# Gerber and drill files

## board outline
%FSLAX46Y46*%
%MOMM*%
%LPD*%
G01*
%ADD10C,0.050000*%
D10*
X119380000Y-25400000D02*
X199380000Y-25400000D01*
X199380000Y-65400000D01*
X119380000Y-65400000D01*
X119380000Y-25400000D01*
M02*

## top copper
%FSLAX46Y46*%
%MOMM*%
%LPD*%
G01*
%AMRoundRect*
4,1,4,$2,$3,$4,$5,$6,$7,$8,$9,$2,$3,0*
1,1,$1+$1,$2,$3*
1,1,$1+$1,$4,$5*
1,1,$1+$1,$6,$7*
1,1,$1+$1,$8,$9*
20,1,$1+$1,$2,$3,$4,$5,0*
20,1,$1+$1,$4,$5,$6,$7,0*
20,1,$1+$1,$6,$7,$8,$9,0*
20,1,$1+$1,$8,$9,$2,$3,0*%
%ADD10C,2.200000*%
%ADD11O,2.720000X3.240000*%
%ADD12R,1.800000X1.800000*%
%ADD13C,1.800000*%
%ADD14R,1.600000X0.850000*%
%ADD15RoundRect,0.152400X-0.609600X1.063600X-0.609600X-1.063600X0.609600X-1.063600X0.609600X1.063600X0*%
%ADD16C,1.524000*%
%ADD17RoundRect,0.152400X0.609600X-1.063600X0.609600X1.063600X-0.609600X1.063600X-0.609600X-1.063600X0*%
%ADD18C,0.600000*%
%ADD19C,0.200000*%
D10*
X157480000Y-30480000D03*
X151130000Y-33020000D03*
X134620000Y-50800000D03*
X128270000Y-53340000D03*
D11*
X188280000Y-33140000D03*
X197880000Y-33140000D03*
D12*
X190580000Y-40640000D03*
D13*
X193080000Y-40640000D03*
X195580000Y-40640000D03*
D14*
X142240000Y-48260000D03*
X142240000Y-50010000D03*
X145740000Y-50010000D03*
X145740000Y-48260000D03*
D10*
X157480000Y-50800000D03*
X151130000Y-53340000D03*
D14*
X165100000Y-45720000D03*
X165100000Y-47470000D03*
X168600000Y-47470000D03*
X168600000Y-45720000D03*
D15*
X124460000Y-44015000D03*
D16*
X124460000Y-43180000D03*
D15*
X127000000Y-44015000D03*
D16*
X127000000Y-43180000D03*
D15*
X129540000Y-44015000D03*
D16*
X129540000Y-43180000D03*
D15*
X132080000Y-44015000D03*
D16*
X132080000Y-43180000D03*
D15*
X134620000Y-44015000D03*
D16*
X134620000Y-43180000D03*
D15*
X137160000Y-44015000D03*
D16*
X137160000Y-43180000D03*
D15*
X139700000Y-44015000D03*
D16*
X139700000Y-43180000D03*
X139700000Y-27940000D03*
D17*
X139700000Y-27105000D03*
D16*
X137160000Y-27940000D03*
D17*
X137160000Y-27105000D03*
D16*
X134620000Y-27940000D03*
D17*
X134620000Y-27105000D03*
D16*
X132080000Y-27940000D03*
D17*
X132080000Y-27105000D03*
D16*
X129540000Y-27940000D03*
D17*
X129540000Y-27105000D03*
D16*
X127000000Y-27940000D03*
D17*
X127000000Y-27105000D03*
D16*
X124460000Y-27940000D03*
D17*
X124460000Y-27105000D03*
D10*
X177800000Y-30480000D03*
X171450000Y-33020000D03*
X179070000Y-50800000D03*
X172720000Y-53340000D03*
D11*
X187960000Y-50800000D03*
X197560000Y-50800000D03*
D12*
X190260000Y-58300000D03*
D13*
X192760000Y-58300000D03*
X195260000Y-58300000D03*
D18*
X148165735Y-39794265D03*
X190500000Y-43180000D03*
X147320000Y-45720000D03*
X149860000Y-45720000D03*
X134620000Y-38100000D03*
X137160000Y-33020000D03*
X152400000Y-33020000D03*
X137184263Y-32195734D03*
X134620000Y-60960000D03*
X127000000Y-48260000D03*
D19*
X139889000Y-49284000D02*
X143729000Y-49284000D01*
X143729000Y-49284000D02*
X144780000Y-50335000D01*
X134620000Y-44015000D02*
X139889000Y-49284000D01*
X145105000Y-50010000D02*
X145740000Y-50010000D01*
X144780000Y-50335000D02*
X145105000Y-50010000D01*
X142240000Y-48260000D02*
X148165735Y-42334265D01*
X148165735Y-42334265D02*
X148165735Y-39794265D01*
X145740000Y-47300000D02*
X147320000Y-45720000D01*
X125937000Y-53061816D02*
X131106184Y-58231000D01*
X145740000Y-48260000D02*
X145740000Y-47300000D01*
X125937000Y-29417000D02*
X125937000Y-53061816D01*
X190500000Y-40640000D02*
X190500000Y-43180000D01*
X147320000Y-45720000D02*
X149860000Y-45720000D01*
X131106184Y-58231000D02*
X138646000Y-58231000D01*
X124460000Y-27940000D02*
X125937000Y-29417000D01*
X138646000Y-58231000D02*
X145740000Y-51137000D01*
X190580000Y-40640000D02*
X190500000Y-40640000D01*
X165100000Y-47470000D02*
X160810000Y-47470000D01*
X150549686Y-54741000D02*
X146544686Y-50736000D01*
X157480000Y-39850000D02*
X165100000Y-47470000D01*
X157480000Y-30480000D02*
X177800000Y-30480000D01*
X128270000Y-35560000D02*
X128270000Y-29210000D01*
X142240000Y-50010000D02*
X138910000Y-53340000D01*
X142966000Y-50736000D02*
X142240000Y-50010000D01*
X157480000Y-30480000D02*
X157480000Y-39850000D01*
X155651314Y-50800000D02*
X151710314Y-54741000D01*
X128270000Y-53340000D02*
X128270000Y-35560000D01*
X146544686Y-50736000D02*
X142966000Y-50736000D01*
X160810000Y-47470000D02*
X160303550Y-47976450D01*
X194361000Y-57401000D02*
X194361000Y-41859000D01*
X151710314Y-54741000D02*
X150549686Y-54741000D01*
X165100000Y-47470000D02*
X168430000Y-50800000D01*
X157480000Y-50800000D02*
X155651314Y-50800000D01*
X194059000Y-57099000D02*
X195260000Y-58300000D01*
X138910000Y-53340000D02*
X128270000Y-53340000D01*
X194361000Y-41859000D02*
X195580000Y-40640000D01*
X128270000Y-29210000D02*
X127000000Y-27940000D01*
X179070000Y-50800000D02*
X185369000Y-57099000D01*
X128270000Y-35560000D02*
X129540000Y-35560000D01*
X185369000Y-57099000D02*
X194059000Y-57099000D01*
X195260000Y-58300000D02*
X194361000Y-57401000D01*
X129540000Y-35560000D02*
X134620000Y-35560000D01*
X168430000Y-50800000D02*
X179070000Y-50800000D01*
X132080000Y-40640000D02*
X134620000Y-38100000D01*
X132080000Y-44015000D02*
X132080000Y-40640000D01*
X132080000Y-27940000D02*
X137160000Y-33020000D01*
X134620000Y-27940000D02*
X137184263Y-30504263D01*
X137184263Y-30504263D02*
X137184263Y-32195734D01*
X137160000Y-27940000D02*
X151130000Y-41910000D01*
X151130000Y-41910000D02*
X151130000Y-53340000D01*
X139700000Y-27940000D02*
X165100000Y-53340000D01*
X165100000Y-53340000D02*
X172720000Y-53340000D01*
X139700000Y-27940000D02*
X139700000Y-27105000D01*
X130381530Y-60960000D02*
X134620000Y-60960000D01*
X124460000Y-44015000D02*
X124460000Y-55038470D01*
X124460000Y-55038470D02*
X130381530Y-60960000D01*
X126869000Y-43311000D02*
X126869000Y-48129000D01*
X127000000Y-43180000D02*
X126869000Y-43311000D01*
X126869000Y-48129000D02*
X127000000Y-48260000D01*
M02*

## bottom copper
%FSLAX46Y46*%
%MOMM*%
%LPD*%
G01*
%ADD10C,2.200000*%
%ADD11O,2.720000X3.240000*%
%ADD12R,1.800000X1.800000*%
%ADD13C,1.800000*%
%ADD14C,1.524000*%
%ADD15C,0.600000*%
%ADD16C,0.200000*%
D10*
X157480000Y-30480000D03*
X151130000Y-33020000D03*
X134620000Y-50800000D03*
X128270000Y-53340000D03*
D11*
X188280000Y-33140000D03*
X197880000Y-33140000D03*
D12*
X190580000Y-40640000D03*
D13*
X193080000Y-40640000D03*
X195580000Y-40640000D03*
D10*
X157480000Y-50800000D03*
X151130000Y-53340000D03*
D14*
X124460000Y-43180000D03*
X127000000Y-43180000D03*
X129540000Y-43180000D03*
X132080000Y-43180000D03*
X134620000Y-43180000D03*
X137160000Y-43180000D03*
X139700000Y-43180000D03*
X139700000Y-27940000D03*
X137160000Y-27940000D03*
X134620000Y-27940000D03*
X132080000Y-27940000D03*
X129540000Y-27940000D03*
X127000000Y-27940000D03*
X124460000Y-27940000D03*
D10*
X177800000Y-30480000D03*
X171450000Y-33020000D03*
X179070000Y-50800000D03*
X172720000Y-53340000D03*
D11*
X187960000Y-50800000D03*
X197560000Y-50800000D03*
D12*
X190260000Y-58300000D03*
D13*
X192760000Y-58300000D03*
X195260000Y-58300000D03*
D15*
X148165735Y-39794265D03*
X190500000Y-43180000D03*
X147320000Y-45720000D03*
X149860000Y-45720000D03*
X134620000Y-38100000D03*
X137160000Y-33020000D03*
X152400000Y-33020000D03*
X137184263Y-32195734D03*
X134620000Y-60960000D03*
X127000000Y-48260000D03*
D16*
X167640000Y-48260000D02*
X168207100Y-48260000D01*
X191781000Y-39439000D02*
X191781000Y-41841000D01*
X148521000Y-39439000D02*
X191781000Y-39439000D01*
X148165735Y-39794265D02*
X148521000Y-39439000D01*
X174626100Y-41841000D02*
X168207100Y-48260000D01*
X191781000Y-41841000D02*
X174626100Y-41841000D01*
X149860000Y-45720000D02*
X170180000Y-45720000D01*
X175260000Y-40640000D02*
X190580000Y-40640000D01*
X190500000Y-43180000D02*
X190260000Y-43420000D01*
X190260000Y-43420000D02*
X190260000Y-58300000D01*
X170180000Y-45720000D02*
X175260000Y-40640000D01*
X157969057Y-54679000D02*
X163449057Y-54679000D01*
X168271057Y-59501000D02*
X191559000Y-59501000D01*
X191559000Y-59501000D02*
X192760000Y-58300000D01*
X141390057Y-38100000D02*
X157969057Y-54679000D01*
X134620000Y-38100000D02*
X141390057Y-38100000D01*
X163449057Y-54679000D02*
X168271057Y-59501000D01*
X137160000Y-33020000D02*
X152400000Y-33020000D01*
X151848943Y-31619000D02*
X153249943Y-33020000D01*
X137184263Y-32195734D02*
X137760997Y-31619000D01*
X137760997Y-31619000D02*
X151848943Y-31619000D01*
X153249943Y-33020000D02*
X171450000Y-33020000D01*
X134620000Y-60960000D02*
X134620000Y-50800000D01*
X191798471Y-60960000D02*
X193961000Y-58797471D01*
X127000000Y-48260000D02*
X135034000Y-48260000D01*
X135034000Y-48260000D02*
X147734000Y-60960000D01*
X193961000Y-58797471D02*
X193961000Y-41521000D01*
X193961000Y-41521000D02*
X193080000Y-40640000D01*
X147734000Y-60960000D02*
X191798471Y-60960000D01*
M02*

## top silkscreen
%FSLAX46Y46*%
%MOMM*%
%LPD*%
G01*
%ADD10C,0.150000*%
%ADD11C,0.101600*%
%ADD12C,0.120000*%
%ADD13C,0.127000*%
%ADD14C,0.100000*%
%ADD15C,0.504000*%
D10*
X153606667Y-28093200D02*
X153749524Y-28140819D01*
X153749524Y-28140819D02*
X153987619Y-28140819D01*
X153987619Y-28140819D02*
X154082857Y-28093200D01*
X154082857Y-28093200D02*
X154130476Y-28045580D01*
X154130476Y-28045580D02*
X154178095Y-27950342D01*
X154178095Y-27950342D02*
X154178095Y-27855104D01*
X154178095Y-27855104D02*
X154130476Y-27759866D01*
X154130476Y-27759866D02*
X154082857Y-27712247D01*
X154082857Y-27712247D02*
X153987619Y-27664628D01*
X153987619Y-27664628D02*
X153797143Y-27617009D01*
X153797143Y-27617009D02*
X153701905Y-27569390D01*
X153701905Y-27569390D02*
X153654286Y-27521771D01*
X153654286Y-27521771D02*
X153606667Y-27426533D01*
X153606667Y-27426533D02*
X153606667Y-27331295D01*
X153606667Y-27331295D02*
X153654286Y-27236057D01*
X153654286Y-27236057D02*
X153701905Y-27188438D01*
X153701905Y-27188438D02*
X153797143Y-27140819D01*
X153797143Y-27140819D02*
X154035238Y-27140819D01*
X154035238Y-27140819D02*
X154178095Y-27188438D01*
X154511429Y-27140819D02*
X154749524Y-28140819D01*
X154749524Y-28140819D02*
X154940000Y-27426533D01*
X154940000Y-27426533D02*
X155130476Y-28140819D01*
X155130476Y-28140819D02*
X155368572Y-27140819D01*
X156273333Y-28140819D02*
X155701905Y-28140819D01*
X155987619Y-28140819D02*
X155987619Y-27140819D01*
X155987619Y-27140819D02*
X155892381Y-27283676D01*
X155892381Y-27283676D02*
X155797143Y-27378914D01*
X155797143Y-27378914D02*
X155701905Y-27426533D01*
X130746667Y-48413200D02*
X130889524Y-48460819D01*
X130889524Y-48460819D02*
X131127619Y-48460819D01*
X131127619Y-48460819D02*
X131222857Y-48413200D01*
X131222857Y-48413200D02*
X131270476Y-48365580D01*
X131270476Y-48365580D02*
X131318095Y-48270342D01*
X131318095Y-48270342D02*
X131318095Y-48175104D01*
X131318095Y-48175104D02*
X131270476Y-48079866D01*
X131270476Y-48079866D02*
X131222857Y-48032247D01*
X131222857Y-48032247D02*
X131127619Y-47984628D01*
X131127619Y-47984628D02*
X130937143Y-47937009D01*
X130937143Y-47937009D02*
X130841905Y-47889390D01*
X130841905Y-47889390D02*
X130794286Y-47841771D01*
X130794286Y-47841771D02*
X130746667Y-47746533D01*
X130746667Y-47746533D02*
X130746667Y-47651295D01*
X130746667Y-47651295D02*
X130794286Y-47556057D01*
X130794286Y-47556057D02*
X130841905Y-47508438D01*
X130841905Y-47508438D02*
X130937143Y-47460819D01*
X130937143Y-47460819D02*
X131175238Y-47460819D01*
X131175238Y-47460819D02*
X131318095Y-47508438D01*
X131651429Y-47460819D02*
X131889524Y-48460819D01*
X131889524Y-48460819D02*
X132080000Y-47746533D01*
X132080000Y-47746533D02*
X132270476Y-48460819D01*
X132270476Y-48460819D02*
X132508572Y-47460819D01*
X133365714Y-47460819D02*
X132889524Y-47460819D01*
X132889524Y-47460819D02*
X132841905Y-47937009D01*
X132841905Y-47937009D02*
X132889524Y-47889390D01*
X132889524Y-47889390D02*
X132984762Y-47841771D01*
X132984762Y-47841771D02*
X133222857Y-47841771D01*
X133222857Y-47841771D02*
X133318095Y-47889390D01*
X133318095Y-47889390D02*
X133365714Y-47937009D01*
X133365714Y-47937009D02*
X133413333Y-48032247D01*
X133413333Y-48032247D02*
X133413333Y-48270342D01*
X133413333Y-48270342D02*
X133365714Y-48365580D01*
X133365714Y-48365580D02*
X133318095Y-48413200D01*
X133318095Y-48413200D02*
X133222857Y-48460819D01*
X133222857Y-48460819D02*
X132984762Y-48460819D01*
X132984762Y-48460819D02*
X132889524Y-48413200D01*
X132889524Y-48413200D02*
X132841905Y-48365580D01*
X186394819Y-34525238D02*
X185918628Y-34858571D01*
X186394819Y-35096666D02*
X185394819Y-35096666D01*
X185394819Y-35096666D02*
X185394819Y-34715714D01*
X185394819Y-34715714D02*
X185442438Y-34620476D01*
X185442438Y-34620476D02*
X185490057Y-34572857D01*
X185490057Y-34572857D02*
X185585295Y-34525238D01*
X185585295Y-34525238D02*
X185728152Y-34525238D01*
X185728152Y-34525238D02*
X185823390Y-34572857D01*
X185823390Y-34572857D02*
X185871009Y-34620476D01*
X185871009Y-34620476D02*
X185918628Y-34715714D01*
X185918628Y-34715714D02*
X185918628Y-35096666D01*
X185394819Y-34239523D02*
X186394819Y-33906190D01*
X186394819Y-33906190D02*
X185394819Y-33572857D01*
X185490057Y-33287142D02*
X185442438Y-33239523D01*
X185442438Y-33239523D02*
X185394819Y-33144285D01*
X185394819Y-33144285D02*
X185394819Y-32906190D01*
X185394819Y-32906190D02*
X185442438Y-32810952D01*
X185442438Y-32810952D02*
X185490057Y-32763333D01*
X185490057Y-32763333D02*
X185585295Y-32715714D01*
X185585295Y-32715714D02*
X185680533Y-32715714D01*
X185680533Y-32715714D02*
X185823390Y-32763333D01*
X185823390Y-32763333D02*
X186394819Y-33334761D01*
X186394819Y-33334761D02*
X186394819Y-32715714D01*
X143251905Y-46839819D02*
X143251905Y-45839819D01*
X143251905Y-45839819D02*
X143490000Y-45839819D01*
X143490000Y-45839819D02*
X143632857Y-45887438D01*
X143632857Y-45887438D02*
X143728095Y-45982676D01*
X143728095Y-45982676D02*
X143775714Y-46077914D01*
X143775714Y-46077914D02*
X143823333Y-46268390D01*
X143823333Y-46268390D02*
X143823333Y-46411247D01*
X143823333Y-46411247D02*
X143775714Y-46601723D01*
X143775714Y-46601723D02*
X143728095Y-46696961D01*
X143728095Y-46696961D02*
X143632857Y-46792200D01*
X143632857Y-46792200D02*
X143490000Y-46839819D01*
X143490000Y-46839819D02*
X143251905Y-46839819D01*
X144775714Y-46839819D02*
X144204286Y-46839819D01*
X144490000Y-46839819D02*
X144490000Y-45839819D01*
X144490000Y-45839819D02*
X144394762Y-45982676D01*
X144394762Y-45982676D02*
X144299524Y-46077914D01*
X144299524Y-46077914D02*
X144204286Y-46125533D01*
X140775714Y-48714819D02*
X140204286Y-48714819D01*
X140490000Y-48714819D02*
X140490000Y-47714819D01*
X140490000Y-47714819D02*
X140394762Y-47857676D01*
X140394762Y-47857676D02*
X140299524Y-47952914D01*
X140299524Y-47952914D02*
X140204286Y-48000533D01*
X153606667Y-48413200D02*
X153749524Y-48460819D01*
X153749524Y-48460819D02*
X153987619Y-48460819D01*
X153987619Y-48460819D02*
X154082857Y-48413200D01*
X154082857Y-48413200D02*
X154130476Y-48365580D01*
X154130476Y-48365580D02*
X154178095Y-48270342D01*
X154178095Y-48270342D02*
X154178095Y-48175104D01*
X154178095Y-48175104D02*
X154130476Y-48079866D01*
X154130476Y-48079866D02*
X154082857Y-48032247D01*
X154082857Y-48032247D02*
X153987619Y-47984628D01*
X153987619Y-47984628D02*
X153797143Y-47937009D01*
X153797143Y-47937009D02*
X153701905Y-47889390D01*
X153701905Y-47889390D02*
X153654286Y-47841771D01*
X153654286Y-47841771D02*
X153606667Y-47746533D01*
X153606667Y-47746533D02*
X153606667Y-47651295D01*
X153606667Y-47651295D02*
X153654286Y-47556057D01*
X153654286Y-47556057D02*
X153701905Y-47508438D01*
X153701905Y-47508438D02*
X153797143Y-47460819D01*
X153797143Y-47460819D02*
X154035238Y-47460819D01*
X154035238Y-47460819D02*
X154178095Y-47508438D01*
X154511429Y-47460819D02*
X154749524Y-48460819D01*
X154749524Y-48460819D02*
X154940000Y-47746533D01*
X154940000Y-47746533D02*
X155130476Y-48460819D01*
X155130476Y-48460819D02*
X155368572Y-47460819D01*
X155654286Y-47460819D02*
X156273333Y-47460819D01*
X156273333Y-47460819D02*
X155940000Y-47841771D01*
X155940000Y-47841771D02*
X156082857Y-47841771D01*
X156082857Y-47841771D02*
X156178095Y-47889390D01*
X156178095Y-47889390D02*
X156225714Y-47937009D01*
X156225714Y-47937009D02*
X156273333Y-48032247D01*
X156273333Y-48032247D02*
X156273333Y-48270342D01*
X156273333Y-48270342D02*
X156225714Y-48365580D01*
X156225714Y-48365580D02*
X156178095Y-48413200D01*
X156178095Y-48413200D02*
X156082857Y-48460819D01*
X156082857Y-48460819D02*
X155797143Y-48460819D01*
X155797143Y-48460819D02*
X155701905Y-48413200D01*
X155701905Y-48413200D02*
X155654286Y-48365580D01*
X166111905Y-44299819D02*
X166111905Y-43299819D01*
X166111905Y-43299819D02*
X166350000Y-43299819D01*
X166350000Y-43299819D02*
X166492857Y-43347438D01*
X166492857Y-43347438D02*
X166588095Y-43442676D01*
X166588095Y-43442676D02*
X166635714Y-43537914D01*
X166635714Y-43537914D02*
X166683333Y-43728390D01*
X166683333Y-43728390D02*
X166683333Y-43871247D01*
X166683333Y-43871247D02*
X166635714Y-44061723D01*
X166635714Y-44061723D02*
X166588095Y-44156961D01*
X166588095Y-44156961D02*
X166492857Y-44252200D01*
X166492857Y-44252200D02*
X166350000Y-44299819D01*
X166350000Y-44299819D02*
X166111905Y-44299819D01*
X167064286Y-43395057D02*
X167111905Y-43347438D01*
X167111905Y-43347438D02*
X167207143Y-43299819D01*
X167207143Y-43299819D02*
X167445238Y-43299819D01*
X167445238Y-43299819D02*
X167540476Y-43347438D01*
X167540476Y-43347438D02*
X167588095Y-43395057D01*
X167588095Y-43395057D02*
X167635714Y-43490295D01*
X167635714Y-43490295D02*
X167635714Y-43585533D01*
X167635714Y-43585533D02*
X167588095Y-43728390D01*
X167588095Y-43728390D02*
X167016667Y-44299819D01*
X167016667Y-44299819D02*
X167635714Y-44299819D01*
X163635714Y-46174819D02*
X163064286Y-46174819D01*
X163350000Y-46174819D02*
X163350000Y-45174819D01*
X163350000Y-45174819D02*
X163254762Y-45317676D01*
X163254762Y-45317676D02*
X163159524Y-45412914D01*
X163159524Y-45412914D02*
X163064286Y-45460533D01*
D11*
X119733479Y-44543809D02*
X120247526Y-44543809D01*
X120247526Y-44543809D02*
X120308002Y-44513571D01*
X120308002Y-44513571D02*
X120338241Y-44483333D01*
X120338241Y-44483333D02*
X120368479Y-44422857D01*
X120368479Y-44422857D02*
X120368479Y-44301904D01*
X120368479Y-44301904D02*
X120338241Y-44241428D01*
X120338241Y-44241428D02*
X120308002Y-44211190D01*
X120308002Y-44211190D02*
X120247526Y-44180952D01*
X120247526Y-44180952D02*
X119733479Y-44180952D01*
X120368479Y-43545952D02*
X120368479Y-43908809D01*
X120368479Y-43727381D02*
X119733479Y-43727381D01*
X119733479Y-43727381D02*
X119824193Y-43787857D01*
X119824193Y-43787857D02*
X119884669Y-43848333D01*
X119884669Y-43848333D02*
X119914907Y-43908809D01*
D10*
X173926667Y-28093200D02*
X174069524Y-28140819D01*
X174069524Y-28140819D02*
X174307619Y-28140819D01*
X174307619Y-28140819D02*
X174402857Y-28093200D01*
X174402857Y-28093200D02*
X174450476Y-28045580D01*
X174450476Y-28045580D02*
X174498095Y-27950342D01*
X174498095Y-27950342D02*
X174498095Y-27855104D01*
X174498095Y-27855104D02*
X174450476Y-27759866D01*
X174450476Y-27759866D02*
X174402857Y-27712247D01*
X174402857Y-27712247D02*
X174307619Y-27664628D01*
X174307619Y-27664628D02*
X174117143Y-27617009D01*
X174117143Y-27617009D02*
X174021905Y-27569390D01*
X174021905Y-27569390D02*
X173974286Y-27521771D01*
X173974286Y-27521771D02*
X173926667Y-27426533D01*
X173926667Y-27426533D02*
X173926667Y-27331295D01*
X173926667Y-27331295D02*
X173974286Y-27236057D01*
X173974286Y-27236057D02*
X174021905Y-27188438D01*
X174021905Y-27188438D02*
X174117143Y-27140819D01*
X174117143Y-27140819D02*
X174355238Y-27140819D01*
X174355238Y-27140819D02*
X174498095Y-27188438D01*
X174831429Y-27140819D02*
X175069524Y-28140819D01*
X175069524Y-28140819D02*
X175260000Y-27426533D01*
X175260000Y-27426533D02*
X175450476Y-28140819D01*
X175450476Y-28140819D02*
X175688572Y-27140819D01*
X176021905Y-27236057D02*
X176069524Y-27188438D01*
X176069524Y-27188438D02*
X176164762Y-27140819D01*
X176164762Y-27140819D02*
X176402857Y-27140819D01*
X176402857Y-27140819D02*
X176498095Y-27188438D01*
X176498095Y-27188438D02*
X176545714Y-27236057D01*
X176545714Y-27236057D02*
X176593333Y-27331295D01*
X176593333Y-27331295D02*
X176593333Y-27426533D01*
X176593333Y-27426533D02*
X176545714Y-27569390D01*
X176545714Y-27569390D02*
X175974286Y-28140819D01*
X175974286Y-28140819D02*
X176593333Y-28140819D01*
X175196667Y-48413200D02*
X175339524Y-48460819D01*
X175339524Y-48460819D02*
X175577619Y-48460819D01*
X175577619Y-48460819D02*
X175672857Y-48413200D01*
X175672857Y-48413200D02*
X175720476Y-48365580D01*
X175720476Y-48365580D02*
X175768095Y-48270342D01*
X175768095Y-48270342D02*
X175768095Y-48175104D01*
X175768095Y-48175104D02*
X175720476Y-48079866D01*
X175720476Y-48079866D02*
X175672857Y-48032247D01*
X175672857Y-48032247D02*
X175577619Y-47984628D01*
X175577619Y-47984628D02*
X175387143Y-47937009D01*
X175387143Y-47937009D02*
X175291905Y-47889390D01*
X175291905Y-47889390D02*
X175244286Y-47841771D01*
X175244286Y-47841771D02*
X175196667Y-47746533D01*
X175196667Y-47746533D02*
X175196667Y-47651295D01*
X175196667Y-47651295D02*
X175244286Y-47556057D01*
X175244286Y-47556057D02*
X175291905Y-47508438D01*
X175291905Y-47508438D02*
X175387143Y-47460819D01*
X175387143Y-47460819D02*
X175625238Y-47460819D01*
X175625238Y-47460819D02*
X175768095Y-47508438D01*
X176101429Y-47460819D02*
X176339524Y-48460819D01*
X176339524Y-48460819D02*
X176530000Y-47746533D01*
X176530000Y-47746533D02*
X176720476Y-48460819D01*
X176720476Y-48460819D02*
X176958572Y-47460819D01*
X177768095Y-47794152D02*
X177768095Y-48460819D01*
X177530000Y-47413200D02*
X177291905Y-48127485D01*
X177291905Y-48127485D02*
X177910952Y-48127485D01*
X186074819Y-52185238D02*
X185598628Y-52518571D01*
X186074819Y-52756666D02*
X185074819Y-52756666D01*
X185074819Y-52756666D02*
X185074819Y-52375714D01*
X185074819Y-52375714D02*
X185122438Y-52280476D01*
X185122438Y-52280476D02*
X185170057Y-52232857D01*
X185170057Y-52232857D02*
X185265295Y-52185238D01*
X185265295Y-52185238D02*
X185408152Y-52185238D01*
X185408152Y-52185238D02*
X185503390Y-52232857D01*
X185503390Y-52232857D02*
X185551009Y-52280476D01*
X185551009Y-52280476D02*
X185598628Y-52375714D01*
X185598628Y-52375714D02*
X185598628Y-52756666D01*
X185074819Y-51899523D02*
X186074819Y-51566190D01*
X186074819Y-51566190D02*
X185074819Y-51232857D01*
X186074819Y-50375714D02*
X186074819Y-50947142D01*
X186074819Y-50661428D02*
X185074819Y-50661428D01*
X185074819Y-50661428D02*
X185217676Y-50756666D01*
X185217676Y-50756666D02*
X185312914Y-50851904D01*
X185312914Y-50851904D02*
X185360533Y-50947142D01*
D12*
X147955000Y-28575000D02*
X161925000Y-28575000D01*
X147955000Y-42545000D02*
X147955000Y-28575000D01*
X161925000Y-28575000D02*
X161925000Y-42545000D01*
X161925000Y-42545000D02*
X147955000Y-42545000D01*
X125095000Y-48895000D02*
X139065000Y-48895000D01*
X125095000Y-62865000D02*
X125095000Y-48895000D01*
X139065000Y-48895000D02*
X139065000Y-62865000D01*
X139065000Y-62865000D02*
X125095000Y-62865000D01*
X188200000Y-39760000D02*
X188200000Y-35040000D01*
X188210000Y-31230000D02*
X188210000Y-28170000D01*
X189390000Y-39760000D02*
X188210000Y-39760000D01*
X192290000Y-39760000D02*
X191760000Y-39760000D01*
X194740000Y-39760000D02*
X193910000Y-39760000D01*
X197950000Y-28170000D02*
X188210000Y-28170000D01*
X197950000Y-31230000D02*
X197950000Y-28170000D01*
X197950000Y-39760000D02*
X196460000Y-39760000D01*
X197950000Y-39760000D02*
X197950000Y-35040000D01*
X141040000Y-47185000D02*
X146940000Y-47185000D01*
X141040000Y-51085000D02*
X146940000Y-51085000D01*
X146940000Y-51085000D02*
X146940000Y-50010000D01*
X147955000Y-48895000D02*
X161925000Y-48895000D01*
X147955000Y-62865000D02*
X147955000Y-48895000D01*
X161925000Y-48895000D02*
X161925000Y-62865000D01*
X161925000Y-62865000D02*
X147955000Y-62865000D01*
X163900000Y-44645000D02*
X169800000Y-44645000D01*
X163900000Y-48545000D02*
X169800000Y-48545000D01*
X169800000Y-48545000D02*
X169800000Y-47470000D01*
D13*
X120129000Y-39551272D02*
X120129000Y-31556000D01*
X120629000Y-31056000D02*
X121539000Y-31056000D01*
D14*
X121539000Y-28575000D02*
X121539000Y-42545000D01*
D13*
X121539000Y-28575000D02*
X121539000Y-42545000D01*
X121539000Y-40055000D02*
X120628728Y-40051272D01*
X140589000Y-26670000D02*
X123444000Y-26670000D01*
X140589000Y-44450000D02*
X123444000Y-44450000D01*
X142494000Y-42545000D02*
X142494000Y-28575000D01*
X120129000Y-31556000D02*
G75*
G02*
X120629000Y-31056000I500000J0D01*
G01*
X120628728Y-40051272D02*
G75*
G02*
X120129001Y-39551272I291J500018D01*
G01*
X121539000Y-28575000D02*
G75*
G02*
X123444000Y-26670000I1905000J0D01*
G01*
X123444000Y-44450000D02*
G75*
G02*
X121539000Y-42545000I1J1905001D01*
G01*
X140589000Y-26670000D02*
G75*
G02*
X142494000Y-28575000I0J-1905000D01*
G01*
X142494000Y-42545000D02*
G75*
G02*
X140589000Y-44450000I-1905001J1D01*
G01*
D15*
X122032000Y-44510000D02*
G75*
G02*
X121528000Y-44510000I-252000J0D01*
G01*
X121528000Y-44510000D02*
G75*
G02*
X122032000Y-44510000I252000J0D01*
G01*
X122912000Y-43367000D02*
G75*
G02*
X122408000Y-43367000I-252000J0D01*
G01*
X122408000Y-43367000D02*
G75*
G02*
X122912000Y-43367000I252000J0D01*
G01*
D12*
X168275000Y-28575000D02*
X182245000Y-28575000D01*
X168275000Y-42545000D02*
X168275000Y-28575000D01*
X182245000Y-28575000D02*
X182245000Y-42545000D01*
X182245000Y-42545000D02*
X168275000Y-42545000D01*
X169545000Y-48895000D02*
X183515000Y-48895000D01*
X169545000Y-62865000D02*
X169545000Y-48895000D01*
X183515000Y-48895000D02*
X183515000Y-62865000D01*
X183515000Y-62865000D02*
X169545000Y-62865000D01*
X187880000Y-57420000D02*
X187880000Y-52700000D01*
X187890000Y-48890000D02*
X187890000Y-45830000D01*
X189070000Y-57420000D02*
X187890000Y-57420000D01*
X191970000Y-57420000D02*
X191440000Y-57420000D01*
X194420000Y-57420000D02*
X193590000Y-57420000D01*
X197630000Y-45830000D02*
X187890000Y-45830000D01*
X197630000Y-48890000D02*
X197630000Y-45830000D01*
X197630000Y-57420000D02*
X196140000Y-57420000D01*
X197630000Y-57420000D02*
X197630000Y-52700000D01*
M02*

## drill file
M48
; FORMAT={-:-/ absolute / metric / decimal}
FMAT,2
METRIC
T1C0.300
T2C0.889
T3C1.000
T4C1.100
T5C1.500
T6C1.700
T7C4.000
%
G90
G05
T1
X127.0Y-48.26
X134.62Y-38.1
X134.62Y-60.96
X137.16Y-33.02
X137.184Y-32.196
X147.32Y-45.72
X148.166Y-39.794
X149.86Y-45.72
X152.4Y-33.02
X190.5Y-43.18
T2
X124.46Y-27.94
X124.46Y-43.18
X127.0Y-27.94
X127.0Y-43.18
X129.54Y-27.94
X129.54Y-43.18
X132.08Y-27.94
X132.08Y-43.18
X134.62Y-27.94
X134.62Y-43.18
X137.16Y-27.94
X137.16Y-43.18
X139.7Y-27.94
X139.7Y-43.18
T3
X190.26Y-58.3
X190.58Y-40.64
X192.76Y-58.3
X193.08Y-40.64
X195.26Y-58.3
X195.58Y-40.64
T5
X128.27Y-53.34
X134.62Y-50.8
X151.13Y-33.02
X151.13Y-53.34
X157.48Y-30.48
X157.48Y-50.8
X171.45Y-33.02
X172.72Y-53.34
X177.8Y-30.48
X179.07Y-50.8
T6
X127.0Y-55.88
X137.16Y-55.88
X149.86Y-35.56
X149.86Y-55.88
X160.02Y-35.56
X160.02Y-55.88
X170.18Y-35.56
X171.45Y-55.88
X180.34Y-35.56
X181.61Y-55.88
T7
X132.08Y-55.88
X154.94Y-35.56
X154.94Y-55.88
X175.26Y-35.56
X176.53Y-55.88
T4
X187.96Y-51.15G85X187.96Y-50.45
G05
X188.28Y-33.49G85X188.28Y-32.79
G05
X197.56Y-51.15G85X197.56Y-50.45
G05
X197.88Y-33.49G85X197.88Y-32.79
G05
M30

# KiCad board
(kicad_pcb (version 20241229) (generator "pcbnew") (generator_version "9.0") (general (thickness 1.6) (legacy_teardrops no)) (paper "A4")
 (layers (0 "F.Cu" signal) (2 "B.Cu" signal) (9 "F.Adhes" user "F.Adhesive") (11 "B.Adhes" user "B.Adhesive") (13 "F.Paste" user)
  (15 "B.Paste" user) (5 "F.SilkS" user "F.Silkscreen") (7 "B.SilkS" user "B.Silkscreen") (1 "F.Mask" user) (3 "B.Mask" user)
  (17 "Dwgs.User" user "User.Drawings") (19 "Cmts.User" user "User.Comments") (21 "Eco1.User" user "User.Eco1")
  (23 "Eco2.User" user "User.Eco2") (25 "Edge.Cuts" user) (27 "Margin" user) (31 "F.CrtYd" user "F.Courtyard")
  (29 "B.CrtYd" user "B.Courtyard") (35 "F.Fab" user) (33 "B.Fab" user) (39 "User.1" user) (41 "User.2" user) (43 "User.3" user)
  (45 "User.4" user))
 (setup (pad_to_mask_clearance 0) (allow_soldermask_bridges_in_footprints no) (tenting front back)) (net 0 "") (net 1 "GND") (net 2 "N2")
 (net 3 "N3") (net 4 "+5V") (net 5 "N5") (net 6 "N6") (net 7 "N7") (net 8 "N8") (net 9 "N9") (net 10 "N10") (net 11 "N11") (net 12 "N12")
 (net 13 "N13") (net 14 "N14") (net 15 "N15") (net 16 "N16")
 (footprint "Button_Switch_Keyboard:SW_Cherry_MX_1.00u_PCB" (layer "F.Cu") (at 157.48 30.48)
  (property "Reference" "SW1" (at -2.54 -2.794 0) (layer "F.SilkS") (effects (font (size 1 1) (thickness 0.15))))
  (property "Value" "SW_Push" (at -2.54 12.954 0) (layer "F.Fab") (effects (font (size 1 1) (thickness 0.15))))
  (fp_line (start -9.525 -1.905) (end 4.445 -1.905) (stroke (width 0.12) (type solid)) (layer "F.SilkS"))
  (fp_line (start -9.525 12.065) (end -9.525 -1.905) (stroke (width 0.12) (type solid)) (layer "F.SilkS"))
  (fp_line (start 4.445 -1.905) (end 4.445 12.065) (stroke (width 0.12) (type solid)) (layer "F.SilkS"))
  (fp_line (start 4.445 12.065) (end -9.525 12.065) (stroke (width 0.12) (type solid)) (layer "F.SilkS"))
  (pad "" np_thru_hole circle (at -7.62 5.08) (size 1.7 1.7) (drill 1.7) (layers "*.Cu" "*.Mask"))
  (pad "" np_thru_hole circle (at -2.54 5.08) (size 4 4) (drill 4) (layers "*.Cu" "*.Mask"))
  (pad "" np_thru_hole circle (at 2.54 5.08) (size 1.7 1.7) (drill 1.7) (layers "*.Cu" "*.Mask"))
  (pad "1" thru_hole circle (at 0 0) (size 2.2 2.2) (drill 1.5) (layers "*.Cu" "*.Mask") (remove_unused_layers no) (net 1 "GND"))
  (pad "2" thru_hole circle (at -6.35 2.54) (size 2.2 2.2) (drill 1.5) (layers "*.Cu" "*.Mask") (remove_unused_layers no) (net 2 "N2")))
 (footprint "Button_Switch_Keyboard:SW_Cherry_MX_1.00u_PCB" (layer "F.Cu") (at 134.62 50.8)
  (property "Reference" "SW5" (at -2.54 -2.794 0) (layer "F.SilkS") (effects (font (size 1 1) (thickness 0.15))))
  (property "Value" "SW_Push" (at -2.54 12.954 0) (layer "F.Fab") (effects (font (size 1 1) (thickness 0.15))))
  (fp_line (start -9.525 -1.905) (end 4.445 -1.905) (stroke (width 0.12) (type solid)) (layer "F.SilkS"))
  (fp_line (start -9.525 12.065) (end -9.525 -1.905) (stroke (width 0.12) (type solid)) (layer "F.SilkS"))
  (fp_line (start 4.445 -1.905) (end 4.445 12.065) (stroke (width 0.12) (type solid)) (layer "F.SilkS"))
  (fp_line (start 4.445 12.065) (end -9.525 12.065) (stroke (width 0.12) (type solid)) (layer "F.SilkS"))
  (pad "" np_thru_hole circle (at -7.62 5.08) (size 1.7 1.7) (drill 1.7) (layers "*.Cu" "*.Mask"))
  (pad "" np_thru_hole circle (at -2.54 5.08) (size 4 4) (drill 4) (layers "*.Cu" "*.Mask"))
  (pad "" np_thru_hole circle (at 2.54 5.08) (size 1.7 1.7) (drill 1.7) (layers "*.Cu" "*.Mask"))
  (pad "1" thru_hole circle (at 0 0) (size 2.2 2.2) (drill 1.5) (layers "*.Cu" "*.Mask") (remove_unused_layers no) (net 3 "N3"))
  (pad "2" thru_hole circle (at -6.35 2.54) (size 2.2 2.2) (drill 1.5) (layers "*.Cu" "*.Mask") (remove_unused_layers no) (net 1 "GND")))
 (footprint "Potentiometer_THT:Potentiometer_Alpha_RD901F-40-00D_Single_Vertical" (layer "F.Cu") (at 190.58 40.64 90)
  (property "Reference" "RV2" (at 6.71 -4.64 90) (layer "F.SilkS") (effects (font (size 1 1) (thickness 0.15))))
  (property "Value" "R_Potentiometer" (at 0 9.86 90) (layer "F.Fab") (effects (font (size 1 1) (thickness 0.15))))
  (fp_line (start 0.88 -2.38) (end 5.6 -2.38) (stroke (width 0.12) (type solid)) (layer "F.SilkS"))
  (fp_line (start 9.41 -2.37) (end 12.47 -2.37) (stroke (width 0.12) (type solid)) (layer "F.SilkS"))
  (fp_line (start 0.88 -1.19) (end 0.88 -2.37) (stroke (width 0.12) (type solid)) (layer "F.SilkS"))
  (fp_line (start 0.88 1.71) (end 0.88 1.18) (stroke (width 0.12) (type solid)) (layer "F.SilkS"))
  (fp_line (start 0.88 4.16) (end 0.88 3.33) (stroke (width 0.12) (type solid)) (layer "F.SilkS"))
  (fp_line (start 12.47 7.37) (end 12.47 -2.37) (stroke (width 0.12) (type solid)) (layer "F.SilkS"))
  (fp_line (start 9.41 7.37) (end 12.47 7.37) (stroke (width 0.12) (type solid)) (layer "F.SilkS"))
  (fp_line (start 0.88 7.37) (end 0.88 5.88) (stroke (width 0.12) (type solid)) (layer "F.SilkS"))
  (fp_line (start 0.88 7.37) (end 5.6 7.37) (stroke (width 0.12) (type solid)) (layer "F.SilkS"))
  (pad "" thru_hole oval (at 7.5 -2.3 180) (size 2.72 3.24) (drill oval 1.1 1.8) (layers "*.Cu" "*.Mask") (remove_unused_layers no))
  (pad "" thru_hole oval (at 7.5 7.3 180) (size 2.72 3.24) (drill oval 1.1 1.8) (layers "*.Cu" "*.Mask") (remove_unused_layers no))
  (pad "1" thru_hole rect (at 0 0 180) (size 1.8 1.8) (drill 1) (layers "*.Cu" "*.Mask") (remove_unused_layers no) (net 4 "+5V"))
  (pad "2" thru_hole circle (at 0 2.5 180) (size 1.8 1.8) (drill 1) (layers "*.Cu" "*.Mask") (remove_unused_layers no) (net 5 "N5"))
  (pad "3" thru_hole circle (at 0 5 180) (size 1.8 1.8) (drill 1) (layers "*.Cu" "*.Mask") (remove_unused_layers no) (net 1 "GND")))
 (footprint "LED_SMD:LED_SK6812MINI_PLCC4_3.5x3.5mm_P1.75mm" (layer "F.Cu") (at 143.99 49.135)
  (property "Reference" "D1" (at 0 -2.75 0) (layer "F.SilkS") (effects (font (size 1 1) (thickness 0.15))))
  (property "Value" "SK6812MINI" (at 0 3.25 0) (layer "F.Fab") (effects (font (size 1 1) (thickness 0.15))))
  (fp_line (start -2.95 -1.95) (end 2.95 -1.95) (stroke (width 0.12) (type solid)) (layer "F.SilkS"))
  (fp_line (start -2.95 1.95) (end 2.95 1.95) (stroke (width 0.12) (type solid)) (layer "F.SilkS"))
  (fp_line (start 2.95 1.95) (end 2.95 0.875) (stroke (width 0.12) (type solid)) (layer "F.SilkS"))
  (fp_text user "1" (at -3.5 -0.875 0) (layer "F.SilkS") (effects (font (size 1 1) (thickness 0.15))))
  (pad "1" smd rect (at -1.75 -0.875) (size 1.6 0.85) (layers "F.Cu" "F.Mask" "F.Paste") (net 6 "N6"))
  (pad "2" smd rect (at -1.75 0.875) (size 1.6 0.85) (layers "F.Cu" "F.Mask" "F.Paste") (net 1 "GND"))
  (pad "3" smd rect (at 1.75 0.875) (size 1.6 0.85) (layers "F.Cu" "F.Mask" "F.Paste") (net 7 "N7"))
  (pad "4" smd rect (at 1.75 -0.875) (size 1.6 0.85) (layers "F.Cu" "F.Mask" "F.Paste") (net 4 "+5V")))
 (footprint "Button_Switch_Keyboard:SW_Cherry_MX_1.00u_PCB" (layer "F.Cu") (at 157.48 50.8)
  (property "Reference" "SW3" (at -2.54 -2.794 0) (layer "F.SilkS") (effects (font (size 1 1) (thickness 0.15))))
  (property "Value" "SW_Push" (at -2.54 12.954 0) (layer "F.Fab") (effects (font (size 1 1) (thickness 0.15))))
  (fp_line (start -9.525 -1.905) (end 4.445 -1.905) (stroke (width 0.12) (type solid)) (layer "F.SilkS"))
  (fp_line (start -9.525 12.065) (end -9.525 -1.905) (stroke (width 0.12) (type solid)) (layer "F.SilkS"))
  (fp_line (start 4.445 -1.905) (end 4.445 12.065) (stroke (width 0.12) (type solid)) (layer "F.SilkS"))
  (fp_line (start 4.445 12.065) (end -9.525 12.065) (stroke (width 0.12) (type solid)) (layer "F.SilkS"))
  (pad "" np_thru_hole circle (at -7.62 5.08) (size 1.7 1.7) (drill 1.7) (layers "*.Cu" "*.Mask"))
  (pad "" np_thru_hole circle (at -2.54 5.08) (size 4 4) (drill 4) (layers "*.Cu" "*.Mask"))
  (pad "" np_thru_hole circle (at 2.54 5.08) (size 1.7 1.7) (drill 1.7) (layers "*.Cu" "*.Mask"))
  (pad "1" thru_hole circle (at 0 0) (size 2.2 2.2) (drill 1.5) (layers "*.Cu" "*.Mask") (remove_unused_layers no) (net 1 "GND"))
  (pad "2" thru_hole circle (at -6.35 2.54) (size 2.2 2.2) (drill 1.5) (layers "*.Cu" "*.Mask") (remove_unused_layers no) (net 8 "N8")))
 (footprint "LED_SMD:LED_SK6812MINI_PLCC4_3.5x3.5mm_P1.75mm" (layer "F.Cu") (at 166.85 46.595)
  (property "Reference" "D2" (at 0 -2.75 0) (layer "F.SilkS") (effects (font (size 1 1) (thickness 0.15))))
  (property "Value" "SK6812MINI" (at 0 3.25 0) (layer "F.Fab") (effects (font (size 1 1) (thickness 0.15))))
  (fp_line (start -2.95 -1.95) (end 2.95 -1.95) (stroke (width 0.12) (type solid)) (layer "F.SilkS"))
  (fp_line (start -2.95 1.95) (end 2.95 1.95) (stroke (width 0.12) (type solid)) (layer "F.SilkS"))
  (fp_line (start 2.95 1.95) (end 2.95 0.875) (stroke (width 0.12) (type solid)) (layer "F.SilkS"))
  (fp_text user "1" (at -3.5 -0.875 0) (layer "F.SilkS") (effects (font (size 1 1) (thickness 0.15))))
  (pad "1" smd rect (at -1.75 -0.875) (size 1.6 0.85) (layers "F.Cu" "F.Mask" "F.Paste") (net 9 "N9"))
  (pad "2" smd rect (at -1.75 0.875) (size 1.6 0.85) (layers "F.Cu" "F.Mask" "F.Paste") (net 1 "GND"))
  (pad "3" smd rect (at 1.75 0.875) (size 1.6 0.85) (layers "F.Cu" "F.Mask" "F.Paste") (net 6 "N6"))
  (pad "4" smd rect (at 1.75 -0.875) (size 1.6 0.85) (layers "F.Cu" "F.Mask" "F.Paste") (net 4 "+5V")))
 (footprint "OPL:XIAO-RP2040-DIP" (layer "F.Cu") (at 132.08 35.56 90)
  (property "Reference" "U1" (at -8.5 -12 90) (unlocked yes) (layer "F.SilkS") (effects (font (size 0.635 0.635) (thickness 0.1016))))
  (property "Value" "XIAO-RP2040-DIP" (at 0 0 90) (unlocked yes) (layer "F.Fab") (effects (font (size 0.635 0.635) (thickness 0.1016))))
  (fp_line (start -3.991272 -11.951) (end 4.004 -11.951) (stroke (width 0.127) (type solid)) (layer "F.SilkS"))
  (fp_line (start 4.504 -11.451) (end 4.504 -10.541) (stroke (width 0.127) (type solid)) (layer "F.SilkS"))
  (fp_line (start 6.985 -10.541) (end -6.985 -10.541) (stroke (width 0.1) (type solid)) (layer "F.SilkS"))
  (fp_line (start 6.985 -10.541) (end -6.985 -10.541) (stroke (width 0.127) (type solid)) (layer "F.SilkS"))
  (fp_line (start -4.495 -10.541) (end -4.491272 -11.451272) (stroke (width 0.127) (type solid)) (layer "F.SilkS"))
  (fp_line (start 8.89 8.509) (end 8.89 -8.636) (stroke (width 0.127) (type solid)) (layer "F.SilkS"))
  (fp_line (start -8.89 8.509) (end -8.89 -8.636) (stroke (width 0.127) (type solid)) (layer "F.SilkS"))
  (fp_line (start -6.985 10.414) (end 6.985 10.414) (stroke (width 0.127) (type solid)) (layer "F.SilkS"))
  (fp_arc (start 4.004 -11.951) (mid 4.357553 -11.804553) (end 4.504 -11.451) (stroke (width 0.127) (type default)) (layer "F.SilkS"))
  (fp_arc (start -4.491272 -11.451272) (mid -4.344728 -11.80464) (end -3.991272 -11.951) (stroke (width 0.127) (type default))
   (layer "F.SilkS"))
  (fp_arc (start 6.985 -10.541) (mid 8.332038 -9.983038) (end 8.89 -8.636) (stroke (width 0.127) (type solid)) (layer "F.SilkS"))
  (fp_arc (start -8.89 -8.636) (mid -8.332038 -9.983038) (end -6.985 -10.541) (stroke (width 0.127) (type solid)) (layer "F.SilkS"))
  (fp_arc (start 8.89 8.509) (mid 8.332038 9.856038) (end 6.985 10.414) (stroke (width 0.127) (type solid)) (layer "F.SilkS"))
  (fp_arc (start -6.985 10.414) (mid -8.332038 9.856038) (end -8.89 8.509) (stroke (width 0.127) (type solid)) (layer "F.SilkS"))
  (fp_circle (center -8.95 -10.3) (end -8.95 -10.554) (stroke (width 0.5) (type solid)) (fill yes) (layer "F.SilkS"))
  (fp_circle (center -7.807 -9.42) (end -7.807 -9.674) (stroke (width 0.5) (type solid)) (fill yes) (layer "F.SilkS"))
  (pad "1" smd roundrect (at -8.455 -7.62 270) (size 2.432 1.524) (layers "F.Cu" "F.Mask") (roundrect_rratio 0.1) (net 3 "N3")
   (thermal_bridge_angle 45))
  (pad "1" thru_hole circle (at -7.62 -7.62 270) (size 1.524 1.524) (drill 0.889) (layers "*.Cu" "*.Mask") (remove_unused_layers no)
   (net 3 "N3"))
  (pad "2" smd roundrect (at -8.455 -5.08 270) (size 2.432 1.524) (layers "F.Cu" "F.Mask") (roundrect_rratio 0.1) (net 5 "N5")
   (thermal_bridge_angle 45))
  (pad "2" thru_hole circle (at -7.62 -5.08 270) (size 1.524 1.524) (drill 0.889) (layers "*.Cu" "*.Mask") (remove_unused_layers no)
   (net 5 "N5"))
  (pad "3" smd roundrect (at -8.455 -2.54 270) (size 2.432 1.524) (layers "F.Cu" "F.Mask") (roundrect_rratio 0.1) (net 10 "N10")
   (thermal_bridge_angle 45))
  (pad "3" thru_hole circle (at -7.62 -2.54 270) (size 1.524 1.524) (drill 0.889) (layers "*.Cu" "*.Mask") (remove_unused_layers no)
   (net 10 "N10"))
  (pad "4" smd roundrect (at -8.455 0 270) (size 2.432 1.524) (layers "F.Cu" "F.Mask") (roundrect_rratio 0.1) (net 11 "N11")
   (thermal_bridge_angle 45))
  (pad "4" thru_hole circle (at -7.62 0 270) (size 1.524 1.524) (drill 0.889) (layers "*.Cu" "*.Mask") (remove_unused_layers no)
   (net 11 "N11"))
  (pad "5" smd roundrect (at -8.455 2.54 270) (size 2.432 1.524) (layers "F.Cu" "F.Mask") (roundrect_rratio 0.1) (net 7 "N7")
   (thermal_bridge_angle 45))
  (pad "5" thru_hole circle (at -7.62 2.54 270) (size 1.524 1.524) (drill 0.889) (layers "*.Cu" "*.Mask") (remove_unused_layers no)
   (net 7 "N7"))
  (pad "6" smd roundrect (at -8.455 5.08 270) (size 2.432 1.524) (layers "F.Cu" "F.Mask") (roundrect_rratio 0.1) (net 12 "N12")
   (thermal_bridge_angle 45))
  (pad "6" thru_hole circle (at -7.62 5.08 270) (size 1.524 1.524) (drill 0.889) (layers "*.Cu" "*.Mask") (remove_unused_layers no)
   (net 12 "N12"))
  (pad "7" smd roundrect (at -8.455 7.62 270) (size 2.432 1.524) (layers "F.Cu" "F.Mask") (roundrect_rratio 0.1) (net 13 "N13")
   (thermal_bridge_angle 45))
  (pad "7" thru_hole circle (at -7.62 7.62 270) (size 1.524 1.524) (drill 0.889) (layers "*.Cu" "*.Mask") (remove_unused_layers no)
   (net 13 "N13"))
  (pad "8" thru_hole circle (at 7.62 7.62 90) (size 1.524 1.524) (drill 0.889) (layers "*.Cu" "*.Mask") (remove_unused_layers no)
   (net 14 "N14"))
  (pad "8" smd roundrect (at 8.455 7.62 90) (size 2.432 1.524) (layers "F.Cu" "F.Mask") (roundrect_rratio 0.1) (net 14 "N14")
   (thermal_bridge_angle 45))
  (pad "9" thru_hole circle (at 7.62 5.08 90) (size 1.524 1.524) (drill 0.889) (layers "*.Cu" "*.Mask") (remove_unused_layers no)
   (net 8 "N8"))
  (pad "9" smd roundrect (at 8.455 5.08 90) (size 2.432 1.524) (layers "F.Cu" "F.Mask") (roundrect_rratio 0.1) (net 8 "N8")
   (thermal_bridge_angle 45))
  (pad "10" thru_hole circle (at 7.62 2.54 90) (size 1.524 1.524) (drill 0.889) (layers "*.Cu" "*.Mask") (remove_unused_layers no)
   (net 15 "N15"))
  (pad "10" smd roundrect (at 8.455 2.54 90) (size 2.432 1.524) (layers "F.Cu" "F.Mask") (roundrect_rratio 0.1) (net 15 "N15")
   (thermal_bridge_angle 45))
  (pad "11" thru_hole circle (at 7.62 0 90) (size 1.524 1.524) (drill 0.889) (layers "*.Cu" "*.Mask") (remove_unused_layers no) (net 2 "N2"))
  (pad "11" smd roundrect (at 8.455 0 90) (size 2.432 1.524) (layers "F.Cu" "F.Mask") (roundrect_rratio 0.1) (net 2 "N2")
   (thermal_bridge_angle 45))
  (pad "12" thru_hole circle (at 7.62 -2.54 90) (size 1.524 1.524) (drill 0.889) (layers "*.Cu" "*.Mask") (remove_unused_layers no)
   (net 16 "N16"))
  (pad "12" smd roundrect (at 8.455 -2.54 90) (size 2.432 1.524) (layers "F.Cu" "F.Mask") (roundrect_rratio 0.1) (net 16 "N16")
   (thermal_bridge_angle 45))
  (pad "13" thru_hole circle (at 7.62 -5.08 90) (size 1.524 1.524) (drill 0.889) (layers "*.Cu" "*.Mask") (remove_unused_layers no)
   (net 1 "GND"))
  (pad "13" smd roundrect (at 8.455 -5.08 90) (size 2.432 1.524) (layers "F.Cu" "F.Mask") (roundrect_rratio 0.1) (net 1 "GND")
   (thermal_bridge_angle 45))
  (pad "14" thru_hole circle (at 7.62 -7.62 90) (size 1.524 1.524) (drill 0.889) (layers "*.Cu" "*.Mask") (remove_unused_layers no)
   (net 4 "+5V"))
  (pad "14" smd roundrect (at 8.455 -7.62 90) (size 2.432 1.524) (layers "F.Cu" "F.Mask") (roundrect_rratio 0.1) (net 4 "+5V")
   (thermal_bridge_angle 45)))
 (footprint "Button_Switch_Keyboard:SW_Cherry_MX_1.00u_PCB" (layer "F.Cu") (at 177.8 30.48)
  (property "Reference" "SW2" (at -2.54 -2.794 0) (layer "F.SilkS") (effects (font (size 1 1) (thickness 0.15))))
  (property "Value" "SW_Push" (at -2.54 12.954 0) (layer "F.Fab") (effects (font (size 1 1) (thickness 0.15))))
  (fp_line (start -9.525 -1.905) (end 4.445 -1.905) (stroke (width 0.12) (type solid)) (layer "F.SilkS"))
  (fp_line (start -9.525 12.065) (end -9.525 -1.905) (stroke (width 0.12) (type solid)) (layer "F.SilkS"))
  (fp_line (start 4.445 -1.905) (end 4.445 12.065) (stroke (width 0.12) (type solid)) (layer "F.SilkS"))
  (fp_line (start 4.445 12.065) (end -9.525 12.065) (stroke (width 0.12) (type solid)) (layer "F.SilkS"))
  (pad "" np_thru_hole circle (at -7.62 5.08) (size 1.7 1.7) (drill 1.7) (layers "*.Cu" "*.Mask"))
  (pad "" np_thru_hole circle (at -2.54 5.08) (size 4 4) (drill 4) (layers "*.Cu" "*.Mask"))
  (pad "" np_thru_hole circle (at 2.54 5.08) (size 1.7 1.7) (drill 1.7) (layers "*.Cu" "*.Mask"))
  (pad "1" thru_hole circle (at 0 0) (size 2.2 2.2) (drill 1.5) (layers "*.Cu" "*.Mask") (remove_unused_layers no) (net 1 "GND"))
  (pad "2" thru_hole circle (at -6.35 2.54) (size 2.2 2.2) (drill 1.5) (layers "*.Cu" "*.Mask") (remove_unused_layers no) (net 15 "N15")))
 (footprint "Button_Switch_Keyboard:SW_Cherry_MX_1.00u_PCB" (layer "F.Cu") (at 179.07 50.8)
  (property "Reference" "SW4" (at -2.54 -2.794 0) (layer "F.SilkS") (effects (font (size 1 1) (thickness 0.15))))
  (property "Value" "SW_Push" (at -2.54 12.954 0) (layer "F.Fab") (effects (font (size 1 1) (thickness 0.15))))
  (fp_line (start -9.525 -1.905) (end 4.445 -1.905) (stroke (width 0.12) (type solid)) (layer "F.SilkS"))
  (fp_line (start -9.525 12.065) (end -9.525 -1.905) (stroke (width 0.12) (type solid)) (layer "F.SilkS"))
  (fp_line (start 4.445 -1.905) (end 4.445 12.065) (stroke (width 0.12) (type solid)) (layer "F.SilkS"))
  (fp_line (start 4.445 12.065) (end -9.525 12.065) (stroke (width 0.12) (type solid)) (layer "F.SilkS"))
  (pad "" np_thru_hole circle (at -7.62 5.08) (size 1.7 1.7) (drill 1.7) (layers "*.Cu" "*.Mask"))
  (pad "" np_thru_hole circle (at -2.54 5.08) (size 4 4) (drill 4) (layers "*.Cu" "*.Mask"))
  (pad "" np_thru_hole circle (at 2.54 5.08) (size 1.7 1.7) (drill 1.7) (layers "*.Cu" "*.Mask"))
  (pad "1" thru_hole circle (at 0 0) (size 2.2 2.2) (drill 1.5) (layers "*.Cu" "*.Mask") (remove_unused_layers no) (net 1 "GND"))
  (pad "2" thru_hole circle (at -6.35 2.54) (size 2.2 2.2) (drill 1.5) (layers "*.Cu" "*.Mask") (remove_unused_layers no) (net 14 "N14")))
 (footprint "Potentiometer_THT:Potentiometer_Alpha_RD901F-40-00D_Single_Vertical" (layer "F.Cu") (at 190.26 58.3 90)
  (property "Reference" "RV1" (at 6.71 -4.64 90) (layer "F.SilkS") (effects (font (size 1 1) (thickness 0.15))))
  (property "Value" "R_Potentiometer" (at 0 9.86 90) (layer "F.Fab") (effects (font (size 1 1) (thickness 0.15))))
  (fp_line (start 0.88 -2.38) (end 5.6 -2.38) (stroke (width 0.12) (type solid)) (layer "F.SilkS"))
  (fp_line (start 9.41 -2.37) (end 12.47 -2.37) (stroke (width 0.12) (type solid)) (layer "F.SilkS"))
  (fp_line (start 0.88 -1.19) (end 0.88 -2.37) (stroke (width 0.12) (type solid)) (layer "F.SilkS"))
  (fp_line (start 0.88 1.71) (end 0.88 1.18) (stroke (width 0.12) (type solid)) (layer "F.SilkS"))
  (fp_line (start 0.88 4.16) (end 0.88 3.33) (stroke (width 0.12) (type solid)) (layer "F.SilkS"))
  (fp_line (start 12.47 7.37) (end 12.47 -2.37) (stroke (width 0.12) (type solid)) (layer "F.SilkS"))
  (fp_line (start 9.41 7.37) (end 12.47 7.37) (stroke (width 0.12) (type solid)) (layer "F.SilkS"))
  (fp_line (start 0.88 7.37) (end 0.88 5.88) (stroke (width 0.12) (type solid)) (layer "F.SilkS"))
  (fp_line (start 0.88 7.37) (end 5.6 7.37) (stroke (width 0.12) (type solid)) (layer "F.SilkS"))
  (pad "" thru_hole oval (at 7.5 -2.3 180) (size 2.72 3.24) (drill oval 1.1 1.8) (layers "*.Cu" "*.Mask") (remove_unused_layers no))
  (pad "" thru_hole oval (at 7.5 7.3 180) (size 2.72 3.24) (drill oval 1.1 1.8) (layers "*.Cu" "*.Mask") (remove_unused_layers no))
  (pad "1" thru_hole rect (at 0 0 180) (size 1.8 1.8) (drill 1) (layers "*.Cu" "*.Mask") (remove_unused_layers no) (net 4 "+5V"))
  (pad "2" thru_hole circle (at 0 2.5 180) (size 1.8 1.8) (drill 1) (layers "*.Cu" "*.Mask") (remove_unused_layers no) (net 11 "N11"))
  (pad "3" thru_hole circle (at 0 5 180) (size 1.8 1.8) (drill 1) (layers "*.Cu" "*.Mask") (remove_unused_layers no) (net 1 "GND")))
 (gr_rect (start 119.38 25.4) (end 199.38 65.4) (stroke (width 0.05) (type default)) (fill no) (layer "Edge.Cuts"))
 (segment (start 139.889 49.284) (end 143.729 49.284) (width 0.2) (layer "F.Cu") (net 7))
 (segment (start 143.729 49.284) (end 144.78 50.335) (width 0.2) (layer "F.Cu") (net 7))
 (segment (start 134.62 44.015) (end 139.889 49.284) (width 0.2) (layer "F.Cu") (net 7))
 (segment (start 145.105 50.01) (end 145.74 50.01) (width 0.2) (layer "F.Cu") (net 7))
 (segment (start 144.78 50.335) (end 145.105 50.01) (width 0.2) (layer "F.Cu") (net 7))
 (segment (start 142.24 48.26) (end 148.165735 42.334265) (width 0.2) (layer "F.Cu") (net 6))
 (segment (start 148.165735 42.334265) (end 148.165735 39.794265) (width 0.2) (layer "F.Cu") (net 6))
 (via (at 148.165735 39.794265) (size 0.6) (drill 0.3) (layers "F.Cu" "B.Cu") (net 6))
 (segment (start 167.64 48.26) (end 168.2071 48.26) (width 0.2) (layer "B.Cu") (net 6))
 (segment (start 191.781 39.439) (end 191.781 41.841) (width 0.2) (layer "B.Cu") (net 6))
 (segment (start 148.521 39.439) (end 191.781 39.439) (width 0.2) (layer "B.Cu") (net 6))
 (segment (start 148.165735 39.794265) (end 148.521 39.439) (width 0.2) (layer "B.Cu") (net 6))
 (segment (start 174.6261 41.841) (end 168.2071 48.26) (width 0.2) (layer "B.Cu") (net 6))
 (segment (start 191.781 41.841) (end 174.6261 41.841) (width 0.2) (layer "B.Cu") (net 6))
 (segment (start 145.74 47.3) (end 147.32 45.72) (width 0.2) (layer "F.Cu") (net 4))
 (segment (start 125.937 53.061816) (end 131.106184 58.231) (width 0.2) (layer "F.Cu") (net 4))
 (segment (start 145.74 48.26) (end 145.74 47.3) (width 0.2) (layer "F.Cu") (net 4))
 (segment (start 125.937 29.417) (end 125.937 53.061816) (width 0.2) (layer "F.Cu") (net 4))
 (segment (start 190.5 40.64) (end 190.5 43.18) (width 0.2) (layer "F.Cu") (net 4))
 (segment (start 147.32 45.72) (end 149.86 45.72) (width 0.2) (layer "F.Cu") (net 4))
 (segment (start 131.106184 58.231) (end 138.646 58.231) (width 0.2) (layer "F.Cu") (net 4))
 (segment (start 124.46 27.94) (end 125.937 29.417) (width 0.2) (layer "F.Cu") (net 4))
 (segment (start 138.646 58.231) (end 145.74 51.137) (width 0.2) (layer "F.Cu") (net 4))
 (segment (start 190.58 40.64) (end 190.5 40.64) (width 0.2) (layer "F.Cu") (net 4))
 (via (at 190.5 43.18) (size 0.6) (drill 0.3) (layers "F.Cu" "B.Cu") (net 4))
 (via (at 147.32 45.72) (size 0.6) (drill 0.3) (layers "F.Cu" "B.Cu") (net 4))
 (via (at 149.86 45.72) (size 0.6) (drill 0.3) (layers "F.Cu" "B.Cu") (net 4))
 (segment (start 149.86 45.72) (end 170.18 45.72) (width 0.2) (layer "B.Cu") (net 4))
 (segment (start 175.26 40.64) (end 190.58 40.64) (width 0.2) (layer "B.Cu") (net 4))
 (segment (start 190.5 43.18) (end 190.26 43.42) (width 0.2) (layer "B.Cu") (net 4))
 (segment (start 190.26 43.42) (end 190.26 58.3) (width 0.2) (layer "B.Cu") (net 4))
 (segment (start 170.18 45.72) (end 175.26 40.64) (width 0.2) (layer "B.Cu") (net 4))
 (segment (start 165.1 47.47) (end 160.81 47.47) (width 0.2) (layer "F.Cu") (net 1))
 (segment (start 150.549686 54.741) (end 146.544686 50.736) (width 0.2) (layer "F.Cu") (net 1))
 (segment (start 157.48 39.85) (end 165.1 47.47) (width 0.2) (layer "F.Cu") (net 1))
 (segment (start 157.48 30.48) (end 177.8 30.48) (width 0.2) (layer "F.Cu") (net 1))
 (segment (start 128.27 35.56) (end 128.27 29.21) (width 0.2) (layer "F.Cu") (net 1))
 (segment (start 142.24 50.01) (end 138.91 53.34) (width 0.2) (layer "F.Cu") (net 1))
 (segment (start 142.966 50.736) (end 142.24 50.01) (width 0.2) (layer "F.Cu") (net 1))
 (segment (start 157.48 30.48) (end 157.48 39.85) (width 0.2) (layer "F.Cu") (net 1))
 (segment (start 155.651314 50.8) (end 151.710314 54.741) (width 0.2) (layer "F.Cu") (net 1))
 (segment (start 128.27 53.34) (end 128.27 35.56) (width 0.2) (layer "F.Cu") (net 1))
 (segment (start 146.544686 50.736) (end 142.966 50.736) (width 0.2) (layer "F.Cu") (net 1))
 (segment (start 160.81 47.47) (end 160.30355 47.97645) (width 0.2) (layer "F.Cu") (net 1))
 (segment (start 194.361 57.401) (end 194.361 41.859) (width 0.2) (layer "F.Cu") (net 1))
 (segment (start 151.710314 54.741) (end 150.549686 54.741) (width 0.2) (layer "F.Cu") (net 1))
 (segment (start 165.1 47.47) (end 168.43 50.8) (width 0.2) (layer "F.Cu") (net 1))
 (segment (start 157.48 50.8) (end 155.651314 50.8) (width 0.2) (layer "F.Cu") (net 1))
 (segment (start 194.059 57.099) (end 195.26 58.3) (width 0.2) (layer "F.Cu") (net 1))
 (segment (start 138.91 53.34) (end 128.27 53.34) (width 0.2) (layer "F.Cu") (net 1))
 (segment (start 194.361 41.859) (end 195.58 40.64) (width 0.2) (layer "F.Cu") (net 1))
 (segment (start 128.27 29.21) (end 127 27.94) (width 0.2) (layer "F.Cu") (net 1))
 (segment (start 179.07 50.8) (end 185.369 57.099) (width 0.2) (layer "F.Cu") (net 1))
 (segment (start 128.27 35.56) (end 129.54 35.56) (width 0.2) (layer "F.Cu") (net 1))
 (segment (start 185.369 57.099) (end 194.059 57.099) (width 0.2) (layer "F.Cu") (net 1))
 (segment (start 195.26 58.3) (end 194.361 57.401) (width 0.2) (layer "F.Cu") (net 1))
 (segment (start 129.54 35.56) (end 134.62 35.56) (width 0.2) (layer "F.Cu") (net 1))
 (segment (start 168.43 50.8) (end 179.07 50.8) (width 0.2) (layer "F.Cu") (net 1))
 (segment (start 132.08 40.64) (end 134.62 38.1) (width 0.2) (layer "F.Cu") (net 11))
 (segment (start 132.08 44.015) (end 132.08 40.64) (width 0.2) (layer "F.Cu") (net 11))
 (via (at 134.62 38.1) (size 0.6) (drill 0.3) (layers "F.Cu" "B.Cu") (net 11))
 (segment (start 157.969057 54.679) (end 163.449057 54.679) (width 0.2) (layer "B.Cu") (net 11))
 (segment (start 168.271057 59.501) (end 191.559 59.501) (width 0.2) (layer "B.Cu") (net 11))
 (segment (start 191.559 59.501) (end 192.76 58.3) (width 0.2) (layer "B.Cu") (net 11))
 (segment (start 141.390057 38.1) (end 157.969057 54.679) (width 0.2) (layer "B.Cu") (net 11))
 (segment (start 134.62 38.1) (end 141.390057 38.1) (width 0.2) (layer "B.Cu") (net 11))
 (segment (start 163.449057 54.679) (end 168.271057 59.501) (width 0.2) (layer "B.Cu") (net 11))
 (segment (start 132.08 27.94) (end 137.16 33.02) (width 0.2) (layer "F.Cu") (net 2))
 (via (at 137.16 33.02) (size 0.6) (drill 0.3) (layers "F.Cu" "B.Cu") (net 2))
 (via (at 152.4 33.02) (size 0.6) (drill 0.3) (layers "F.Cu" "B.Cu") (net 2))
 (segment (start 137.16 33.02) (end 152.4 33.02) (width 0.2) (layer "B.Cu") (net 2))
 (segment (start 134.62 27.94) (end 137.184263 30.504263) (width 0.2) (layer "F.Cu") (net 15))
 (segment (start 137.184263 30.504263) (end 137.184263 32.195734) (width 0.2) (layer "F.Cu") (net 15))
 (via (at 137.184263 32.195734) (size 0.6) (drill 0.3) (layers "F.Cu" "B.Cu") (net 15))
 (segment (start 151.848943 31.619) (end 153.249943 33.02) (width 0.2) (layer "B.Cu") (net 15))
 (segment (start 137.184263 32.195734) (end 137.760997 31.619) (width 0.2) (layer "B.Cu") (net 15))
 (segment (start 137.760997 31.619) (end 151.848943 31.619) (width 0.2) (layer "B.Cu") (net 15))
 (segment (start 153.249943 33.02) (end 171.45 33.02) (width 0.2) (layer "B.Cu") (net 15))
 (segment (start 137.16 27.94) (end 151.13 41.91) (width 0.2) (layer "F.Cu") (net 8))
 (segment (start 151.13 41.91) (end 151.13 53.34) (width 0.2) (layer "F.Cu") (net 8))
 (segment (start 139.7 27.94) (end 165.1 53.34) (width 0.2) (layer "F.Cu") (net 14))
 (segment (start 165.1 53.34) (end 172.72 53.34) (width 0.2) (layer "F.Cu") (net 14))
 (segment (start 139.7 27.94) (end 139.7 27.105) (width 0.2) (layer "F.Cu") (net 14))
 (segment (start 130.38153 60.96) (end 134.62 60.96) (width 0.2) (layer "F.Cu") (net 3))
 (segment (start 124.46 44.015) (end 124.46 55.03847) (width 0.2) (layer "F.Cu") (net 3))
 (segment (start 124.46 55.03847) (end 130.38153 60.96) (width 0.2) (layer "F.Cu") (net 3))
 (via (at 134.62 60.96) (size 0.6) (drill 0.3) (layers "F.Cu" "B.Cu") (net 3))
 (segment (start 134.62 60.96) (end 134.62 50.8) (width 0.2) (layer "B.Cu") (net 3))
 (segment (start 126.869 43.311) (end 126.869 48.129) (width 0.2) (layer "F.Cu") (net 5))
 (segment (start 127 43.18) (end 126.869 43.311) (width 0.2) (layer "F.Cu") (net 5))
 (segment (start 126.869 48.129) (end 127 48.26) (width 0.2) (layer "F.Cu") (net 5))
 (via (at 127 48.26) (size 0.6) (drill 0.3) (layers "F.Cu" "B.Cu") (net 5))
 (segment (start 191.798471 60.96) (end 193.961 58.797471) (width 0.2) (layer "B.Cu") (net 5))
 (segment (start 127 48.26) (end 135.034 48.26) (width 0.2) (layer "B.Cu") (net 5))
 (segment (start 135.034 48.26) (end 147.734 60.96) (width 0.2) (layer "B.Cu") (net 5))
 (segment (start 193.961 58.797471) (end 193.961 41.521) (width 0.2) (layer "B.Cu") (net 5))
 (segment (start 193.961 41.521) (end 193.08 40.64) (width 0.2) (layer "B.Cu") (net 5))
 (segment (start 147.734 60.96) (end 191.798471 60.96) (width 0.2) (layer "B.Cu") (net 5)))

